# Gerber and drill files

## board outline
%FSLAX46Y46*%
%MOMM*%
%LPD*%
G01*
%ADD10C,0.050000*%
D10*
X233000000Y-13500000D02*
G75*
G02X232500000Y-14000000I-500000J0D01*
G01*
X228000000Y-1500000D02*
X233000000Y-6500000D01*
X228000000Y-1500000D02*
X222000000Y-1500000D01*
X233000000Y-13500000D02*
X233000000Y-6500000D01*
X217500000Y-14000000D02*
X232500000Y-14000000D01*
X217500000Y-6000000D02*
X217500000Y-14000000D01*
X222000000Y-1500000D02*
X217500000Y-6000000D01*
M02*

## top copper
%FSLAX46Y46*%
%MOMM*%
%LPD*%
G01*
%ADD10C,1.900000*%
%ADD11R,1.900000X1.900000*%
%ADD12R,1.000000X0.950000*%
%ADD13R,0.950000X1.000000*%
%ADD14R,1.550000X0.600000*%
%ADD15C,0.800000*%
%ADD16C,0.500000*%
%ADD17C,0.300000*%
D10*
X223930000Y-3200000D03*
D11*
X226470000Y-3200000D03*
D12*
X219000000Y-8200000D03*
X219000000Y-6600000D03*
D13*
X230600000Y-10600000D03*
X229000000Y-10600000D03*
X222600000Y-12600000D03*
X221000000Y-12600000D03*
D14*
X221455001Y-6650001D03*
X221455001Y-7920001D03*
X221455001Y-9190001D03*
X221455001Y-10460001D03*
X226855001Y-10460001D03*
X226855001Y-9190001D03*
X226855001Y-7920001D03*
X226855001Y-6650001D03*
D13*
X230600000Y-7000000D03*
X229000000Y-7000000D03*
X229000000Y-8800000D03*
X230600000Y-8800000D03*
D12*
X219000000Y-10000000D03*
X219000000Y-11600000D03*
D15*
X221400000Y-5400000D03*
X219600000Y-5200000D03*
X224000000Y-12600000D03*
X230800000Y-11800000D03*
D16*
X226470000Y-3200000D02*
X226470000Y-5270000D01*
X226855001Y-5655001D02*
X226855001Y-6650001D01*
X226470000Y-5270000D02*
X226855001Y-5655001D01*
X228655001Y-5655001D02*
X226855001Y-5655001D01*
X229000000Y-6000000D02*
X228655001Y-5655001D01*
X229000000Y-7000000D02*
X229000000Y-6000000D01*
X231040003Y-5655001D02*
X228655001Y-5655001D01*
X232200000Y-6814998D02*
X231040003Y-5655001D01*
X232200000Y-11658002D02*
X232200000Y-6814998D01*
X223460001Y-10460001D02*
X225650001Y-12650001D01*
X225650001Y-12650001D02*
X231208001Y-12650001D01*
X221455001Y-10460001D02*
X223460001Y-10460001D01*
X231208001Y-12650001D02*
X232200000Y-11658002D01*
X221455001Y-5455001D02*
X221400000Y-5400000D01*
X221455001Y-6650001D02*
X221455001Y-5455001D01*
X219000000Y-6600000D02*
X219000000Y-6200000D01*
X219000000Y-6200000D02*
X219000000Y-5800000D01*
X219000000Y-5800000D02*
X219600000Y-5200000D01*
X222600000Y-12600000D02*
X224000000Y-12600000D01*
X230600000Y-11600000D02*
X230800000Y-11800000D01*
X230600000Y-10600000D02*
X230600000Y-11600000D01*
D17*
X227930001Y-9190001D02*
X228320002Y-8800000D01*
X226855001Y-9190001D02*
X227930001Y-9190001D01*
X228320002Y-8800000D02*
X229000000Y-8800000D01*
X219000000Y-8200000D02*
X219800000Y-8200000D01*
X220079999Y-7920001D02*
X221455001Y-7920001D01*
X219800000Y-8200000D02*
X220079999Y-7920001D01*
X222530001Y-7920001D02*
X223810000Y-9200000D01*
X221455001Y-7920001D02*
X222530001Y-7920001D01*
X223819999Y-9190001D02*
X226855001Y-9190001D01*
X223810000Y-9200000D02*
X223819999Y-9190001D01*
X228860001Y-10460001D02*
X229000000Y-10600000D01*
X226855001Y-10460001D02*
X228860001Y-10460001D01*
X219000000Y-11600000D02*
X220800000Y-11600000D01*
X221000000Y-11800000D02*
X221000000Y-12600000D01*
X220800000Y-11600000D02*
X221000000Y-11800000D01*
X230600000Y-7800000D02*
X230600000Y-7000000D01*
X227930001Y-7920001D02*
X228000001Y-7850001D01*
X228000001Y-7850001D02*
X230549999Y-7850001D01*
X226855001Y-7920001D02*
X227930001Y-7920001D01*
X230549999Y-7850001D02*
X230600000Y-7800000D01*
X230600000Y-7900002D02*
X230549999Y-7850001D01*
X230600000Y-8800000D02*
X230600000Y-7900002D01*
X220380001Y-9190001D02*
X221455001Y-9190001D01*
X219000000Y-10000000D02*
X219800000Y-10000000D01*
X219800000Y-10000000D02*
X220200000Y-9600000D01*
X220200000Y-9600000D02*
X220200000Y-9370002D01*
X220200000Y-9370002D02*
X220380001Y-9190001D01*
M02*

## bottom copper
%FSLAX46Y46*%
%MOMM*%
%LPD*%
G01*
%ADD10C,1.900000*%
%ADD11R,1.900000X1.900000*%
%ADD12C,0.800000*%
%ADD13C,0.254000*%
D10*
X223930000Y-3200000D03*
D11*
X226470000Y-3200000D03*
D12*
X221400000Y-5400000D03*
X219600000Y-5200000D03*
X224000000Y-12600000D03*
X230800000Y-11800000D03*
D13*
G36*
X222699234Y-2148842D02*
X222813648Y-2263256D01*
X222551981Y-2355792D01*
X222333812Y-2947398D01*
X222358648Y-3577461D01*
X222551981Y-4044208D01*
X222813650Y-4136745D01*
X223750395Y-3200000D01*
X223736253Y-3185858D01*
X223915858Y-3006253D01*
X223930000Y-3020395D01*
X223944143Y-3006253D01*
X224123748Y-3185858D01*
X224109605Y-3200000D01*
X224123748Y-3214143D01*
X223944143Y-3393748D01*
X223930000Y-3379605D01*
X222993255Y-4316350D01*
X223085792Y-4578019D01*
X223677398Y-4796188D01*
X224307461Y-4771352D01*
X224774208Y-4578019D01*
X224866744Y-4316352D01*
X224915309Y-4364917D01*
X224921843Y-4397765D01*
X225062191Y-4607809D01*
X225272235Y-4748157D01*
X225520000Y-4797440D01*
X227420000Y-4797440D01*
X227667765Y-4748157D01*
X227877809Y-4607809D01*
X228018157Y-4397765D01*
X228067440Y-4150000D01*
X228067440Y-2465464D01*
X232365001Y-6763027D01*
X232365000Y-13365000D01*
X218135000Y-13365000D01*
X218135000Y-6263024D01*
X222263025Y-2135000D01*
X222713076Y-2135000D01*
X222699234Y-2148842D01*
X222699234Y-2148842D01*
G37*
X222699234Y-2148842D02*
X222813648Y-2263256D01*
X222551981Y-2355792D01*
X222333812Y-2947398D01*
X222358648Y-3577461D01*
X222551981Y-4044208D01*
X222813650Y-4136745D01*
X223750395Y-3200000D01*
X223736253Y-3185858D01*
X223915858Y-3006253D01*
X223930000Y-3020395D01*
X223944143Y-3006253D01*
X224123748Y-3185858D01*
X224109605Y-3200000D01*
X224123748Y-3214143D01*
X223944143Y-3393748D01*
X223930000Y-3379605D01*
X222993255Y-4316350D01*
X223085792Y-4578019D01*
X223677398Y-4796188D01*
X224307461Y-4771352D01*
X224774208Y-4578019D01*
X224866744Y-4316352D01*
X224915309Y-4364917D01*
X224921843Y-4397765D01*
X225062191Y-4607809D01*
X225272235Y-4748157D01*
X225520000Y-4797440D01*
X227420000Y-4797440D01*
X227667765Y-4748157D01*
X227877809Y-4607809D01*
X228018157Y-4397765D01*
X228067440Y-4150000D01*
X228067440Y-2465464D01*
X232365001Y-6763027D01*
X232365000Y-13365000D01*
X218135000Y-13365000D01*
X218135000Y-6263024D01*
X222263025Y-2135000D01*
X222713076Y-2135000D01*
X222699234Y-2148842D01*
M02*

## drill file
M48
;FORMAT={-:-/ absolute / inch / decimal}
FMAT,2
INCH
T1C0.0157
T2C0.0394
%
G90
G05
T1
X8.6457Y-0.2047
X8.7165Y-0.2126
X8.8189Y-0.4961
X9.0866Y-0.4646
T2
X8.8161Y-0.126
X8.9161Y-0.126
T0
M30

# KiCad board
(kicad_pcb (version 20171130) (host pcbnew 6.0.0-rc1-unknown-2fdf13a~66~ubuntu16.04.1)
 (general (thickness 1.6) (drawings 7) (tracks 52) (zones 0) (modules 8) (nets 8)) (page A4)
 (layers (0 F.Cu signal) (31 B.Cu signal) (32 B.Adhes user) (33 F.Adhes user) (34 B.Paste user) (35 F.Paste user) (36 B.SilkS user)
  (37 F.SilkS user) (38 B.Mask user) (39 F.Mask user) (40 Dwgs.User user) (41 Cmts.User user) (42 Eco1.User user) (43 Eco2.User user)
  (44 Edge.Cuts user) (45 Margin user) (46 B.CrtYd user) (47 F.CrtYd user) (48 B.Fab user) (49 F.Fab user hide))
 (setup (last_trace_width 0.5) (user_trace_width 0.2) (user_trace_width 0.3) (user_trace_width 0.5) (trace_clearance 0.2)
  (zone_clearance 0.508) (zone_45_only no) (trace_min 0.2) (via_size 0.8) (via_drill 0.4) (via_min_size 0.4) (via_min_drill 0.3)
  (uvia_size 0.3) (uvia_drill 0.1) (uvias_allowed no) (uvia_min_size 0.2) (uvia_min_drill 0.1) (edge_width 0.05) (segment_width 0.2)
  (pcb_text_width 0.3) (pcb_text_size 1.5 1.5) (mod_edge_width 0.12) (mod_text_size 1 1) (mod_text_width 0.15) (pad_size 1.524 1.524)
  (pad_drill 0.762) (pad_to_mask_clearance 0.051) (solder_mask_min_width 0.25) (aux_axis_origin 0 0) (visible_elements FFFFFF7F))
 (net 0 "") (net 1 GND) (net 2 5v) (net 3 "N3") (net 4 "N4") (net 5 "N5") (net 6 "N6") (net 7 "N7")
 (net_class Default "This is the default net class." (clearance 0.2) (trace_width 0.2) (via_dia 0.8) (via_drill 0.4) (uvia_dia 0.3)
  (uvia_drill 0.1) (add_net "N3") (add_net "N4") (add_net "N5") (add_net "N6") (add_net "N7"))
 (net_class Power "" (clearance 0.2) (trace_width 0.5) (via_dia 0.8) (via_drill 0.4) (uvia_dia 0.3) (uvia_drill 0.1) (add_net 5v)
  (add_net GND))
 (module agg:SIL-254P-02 (layer F.Cu) (at 225.2 3.2 180)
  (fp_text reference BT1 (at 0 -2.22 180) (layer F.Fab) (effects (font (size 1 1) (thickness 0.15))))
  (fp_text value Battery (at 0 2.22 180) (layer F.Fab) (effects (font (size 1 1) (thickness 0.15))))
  (pad 2 thru_hole circle (at 1.27 0 180) (size 1.9 1.9) (drill 1) (layers *.Cu *.Mask F.SilkS) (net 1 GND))
  (pad 1 thru_hole rect (at -1.27 0 180) (size 1.9 1.9) (drill 1) (layers *.Cu *.Mask F.SilkS) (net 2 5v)))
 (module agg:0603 (layer F.Cu) (at 219 7.4 270)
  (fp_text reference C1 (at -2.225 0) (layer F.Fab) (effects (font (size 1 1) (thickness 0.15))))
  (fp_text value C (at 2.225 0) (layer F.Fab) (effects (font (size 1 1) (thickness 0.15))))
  (pad 2 smd rect (at 0.8 0 270) (size 0.95 1) (layers F.Cu F.Paste F.Mask) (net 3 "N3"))
  (pad 1 smd rect (at -0.8 0 270) (size 0.95 1) (layers F.Cu F.Paste F.Mask) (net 1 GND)))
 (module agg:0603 (layer F.Cu) (at 229.8 10.6 180)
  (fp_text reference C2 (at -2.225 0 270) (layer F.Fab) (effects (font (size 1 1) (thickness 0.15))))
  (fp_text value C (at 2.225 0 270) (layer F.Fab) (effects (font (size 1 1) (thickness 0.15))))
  (pad 1 smd rect (at -0.8 0 180) (size 0.95 1) (layers F.Cu F.Paste F.Mask) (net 1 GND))
  (pad 2 smd rect (at 0.8 0 180) (size 0.95 1) (layers F.Cu F.Paste F.Mask) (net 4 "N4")))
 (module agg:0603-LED (layer F.Cu) (at 221.8 12.6 180)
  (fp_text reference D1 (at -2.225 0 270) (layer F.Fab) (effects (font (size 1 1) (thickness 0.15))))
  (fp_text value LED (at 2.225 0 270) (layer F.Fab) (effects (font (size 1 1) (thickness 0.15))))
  (pad 1 smd rect (at -0.8 0 180) (size 0.95 1) (layers F.Cu F.Paste F.Mask) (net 1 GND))
  (pad 2 smd rect (at 0.8 0 180) (size 0.95 1) (layers F.Cu F.Paste F.Mask) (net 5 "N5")))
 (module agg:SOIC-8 (layer F.Cu) (at 224.155001 8.555001)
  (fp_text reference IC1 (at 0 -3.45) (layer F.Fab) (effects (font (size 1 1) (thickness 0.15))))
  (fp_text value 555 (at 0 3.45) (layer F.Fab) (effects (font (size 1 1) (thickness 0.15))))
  (pad 1 smd rect (at -2.7 -1.905) (size 1.55 0.6) (layers F.Cu F.Paste F.Mask) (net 1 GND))
  (pad 2 smd rect (at -2.7 -0.635) (size 1.55 0.6) (layers F.Cu F.Paste F.Mask) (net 3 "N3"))
  (pad 3 smd rect (at -2.7 0.635) (size 1.55 0.6) (layers F.Cu F.Paste F.Mask) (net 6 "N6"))
  (pad 4 smd rect (at -2.7 1.905) (size 1.55 0.6) (layers F.Cu F.Paste F.Mask) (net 2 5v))
  (pad 5 smd rect (at 2.7 1.905) (size 1.55 0.6) (layers F.Cu F.Paste F.Mask) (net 4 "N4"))
  (pad 6 smd rect (at 2.7 0.635) (size 1.55 0.6) (layers F.Cu F.Paste F.Mask) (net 3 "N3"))
  (pad 7 smd rect (at 2.7 -0.635) (size 1.55 0.6) (layers F.Cu F.Paste F.Mask) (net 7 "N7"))
  (pad 8 smd rect (at 2.7 -1.905) (size 1.55 0.6) (layers F.Cu F.Paste F.Mask) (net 2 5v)))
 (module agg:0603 (layer F.Cu) (at 229.8 7)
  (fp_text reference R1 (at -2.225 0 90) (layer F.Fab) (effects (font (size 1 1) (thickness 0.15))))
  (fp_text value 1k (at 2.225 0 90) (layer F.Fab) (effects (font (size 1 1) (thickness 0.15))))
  (pad 2 smd rect (at 0.8 0) (size 0.95 1) (layers F.Cu F.Paste F.Mask) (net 7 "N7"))
  (pad 1 smd rect (at -0.8 0) (size 0.95 1) (layers F.Cu F.Paste F.Mask) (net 2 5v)))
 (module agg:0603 (layer F.Cu) (at 229.8 8.8)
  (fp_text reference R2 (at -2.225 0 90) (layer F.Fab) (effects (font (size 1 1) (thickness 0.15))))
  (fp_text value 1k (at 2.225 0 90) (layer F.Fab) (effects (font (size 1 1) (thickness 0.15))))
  (pad 1 smd rect (at -0.8 0) (size 0.95 1) (layers F.Cu F.Paste F.Mask) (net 3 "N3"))
  (pad 2 smd rect (at 0.8 0) (size 0.95 1) (layers F.Cu F.Paste F.Mask) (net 7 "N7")))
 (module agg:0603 (layer F.Cu) (at 219 10.8 270)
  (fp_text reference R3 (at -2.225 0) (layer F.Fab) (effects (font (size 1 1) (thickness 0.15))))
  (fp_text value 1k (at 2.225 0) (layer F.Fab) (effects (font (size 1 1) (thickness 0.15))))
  (pad 1 smd rect (at -0.8 0 270) (size 0.95 1) (layers F.Cu F.Paste F.Mask) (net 6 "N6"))
  (pad 2 smd rect (at 0.8 0 270) (size 0.95 1) (layers F.Cu F.Paste F.Mask) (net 5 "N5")))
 (gr_arc (start 232.5 13.5) (end 232.5 14) (angle -90) (layer Edge.Cuts) (width 0.05))
 (gr_line (start 228 1.5) (end 233 6.5) (layer Edge.Cuts) (width 0.05))
 (gr_line (start 228 1.5) (end 222 1.5) (layer Edge.Cuts) (width 0.05))
 (gr_line (start 233 13.5) (end 233 6.5) (layer Edge.Cuts) (width 0.05))
 (gr_line (start 217.5 14) (end 232.5 14) (layer Edge.Cuts) (width 0.05))
 (gr_line (start 217.5 6) (end 217.5 14) (layer Edge.Cuts) (width 0.05))
 (gr_line (start 222 1.5) (end 217.5 6) (layer Edge.Cuts) (width 0.05))
 (segment (start 226.47 3.2) (end 226.47 5.27) (width 0.5) (layer F.Cu) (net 2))
 (segment (start 226.855001 5.655001) (end 226.855001 6.650001) (width 0.5) (layer F.Cu) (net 2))
 (segment (start 226.47 5.27) (end 226.855001 5.655001) (width 0.5) (layer F.Cu) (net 2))
 (segment (start 228.655001 5.655001) (end 226.855001 5.655001) (width 0.5) (layer F.Cu) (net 2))
 (segment (start 229 6) (end 228.655001 5.655001) (width 0.5) (layer F.Cu) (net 2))
 (segment (start 229 7) (end 229 6) (width 0.5) (layer F.Cu) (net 2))
 (segment (start 231.040003 5.655001) (end 228.655001 5.655001) (width 0.5) (layer F.Cu) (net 2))
 (segment (start 232.2 6.814998) (end 231.040003 5.655001) (width 0.5) (layer F.Cu) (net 2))
 (segment (start 232.2 11.658002) (end 232.2 6.814998) (width 0.5) (layer F.Cu) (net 2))
 (segment (start 223.460001 10.460001) (end 225.650001 12.650001) (width 0.5) (layer F.Cu) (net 2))
 (segment (start 225.650001 12.650001) (end 231.208001 12.650001) (width 0.5) (layer F.Cu) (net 2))
 (segment (start 221.455001 10.460001) (end 223.460001 10.460001) (width 0.5) (layer F.Cu) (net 2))
 (segment (start 231.208001 12.650001) (end 232.2 11.658002) (width 0.5) (layer F.Cu) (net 2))
 (segment (start 221.455001 5.455001) (end 221.4 5.4) (width 0.5) (layer F.Cu) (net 1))
 (via (at 221.4 5.4) (size 0.8) (drill 0.4) (layers F.Cu B.Cu) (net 1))
 (segment (start 221.455001 6.650001) (end 221.455001 5.455001) (width 0.5) (layer F.Cu) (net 1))
 (segment (start 219 6.6) (end 219 6.2) (width 0.5) (layer F.Cu) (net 1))
 (segment (start 219 6.2) (end 219 5.8) (width 0.5) (layer F.Cu) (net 1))
 (segment (start 219 5.8) (end 219.6 5.2) (width 0.5) (layer F.Cu) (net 1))
 (via (at 219.6 5.2) (size 0.8) (drill 0.4) (layers F.Cu B.Cu) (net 1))
 (via (at 224 12.6) (size 0.8) (drill 0.4) (layers F.Cu B.Cu) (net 1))
 (segment (start 222.6 12.6) (end 224 12.6) (width 0.5) (layer F.Cu) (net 1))
 (via (at 230.8 11.8) (size 0.8) (drill 0.4) (layers F.Cu B.Cu) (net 1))
 (segment (start 230.6 11.6) (end 230.8 11.8) (width 0.5) (layer F.Cu) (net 1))
 (segment (start 230.6 10.6) (end 230.6 11.6) (width 0.5) (layer F.Cu) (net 1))
 (segment (start 227.930001 9.190001) (end 228.320002 8.8) (width 0.3) (layer F.Cu) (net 3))
 (segment (start 226.855001 9.190001) (end 227.930001 9.190001) (width 0.3) (layer F.Cu) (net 3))
 (segment (start 228.320002 8.8) (end 229 8.8) (width 0.3) (layer F.Cu) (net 3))
 (segment (start 219 8.2) (end 219.8 8.2) (width 0.3) (layer F.Cu) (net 3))
 (segment (start 220.079999 7.920001) (end 221.455001 7.920001) (width 0.3) (layer F.Cu) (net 3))
 (segment (start 219.8 8.2) (end 220.079999 7.920001) (width 0.3) (layer F.Cu) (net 3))
 (segment (start 222.530001 7.920001) (end 223.81 9.2) (width 0.3) (layer F.Cu) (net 3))
 (segment (start 221.455001 7.920001) (end 222.530001 7.920001) (width 0.3) (layer F.Cu) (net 3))
 (segment (start 223.819999 9.190001) (end 226.855001 9.190001) (width 0.3) (layer F.Cu) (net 3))
 (segment (start 223.81 9.2) (end 223.819999 9.190001) (width 0.3) (layer F.Cu) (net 3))
 (segment (start 228.860001 10.460001) (end 229 10.6) (width 0.3) (layer F.Cu) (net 4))
 (segment (start 226.855001 10.460001) (end 228.860001 10.460001) (width 0.3) (layer F.Cu) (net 4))
 (segment (start 219 11.6) (end 220.8 11.6) (width 0.3) (layer F.Cu) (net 5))
 (segment (start 221 11.8) (end 221 12.6) (width 0.3) (layer F.Cu) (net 5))
 (segment (start 220.8 11.6) (end 221 11.8) (width 0.3) (layer F.Cu) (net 5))
 (segment (start 230.6 7.8) (end 230.6 7) (width 0.3) (layer F.Cu) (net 7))
 (segment (start 227.930001 7.920001) (end 228.000001 7.850001) (width 0.3) (layer F.Cu) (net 7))
 (segment (start 228.000001 7.850001) (end 230.549999 7.850001) (width 0.3) (layer F.Cu) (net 7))
 (segment (start 226.855001 7.920001) (end 227.930001 7.920001) (width 0.3) (layer F.Cu) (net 7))
 (segment (start 230.549999 7.850001) (end 230.6 7.8) (width 0.3) (layer F.Cu) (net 7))
 (segment (start 230.6 7.900002) (end 230.549999 7.850001) (width 0.3) (layer F.Cu) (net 7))
 (segment (start 230.6 8.8) (end 230.6 7.900002) (width 0.3) (layer F.Cu) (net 7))
 (segment (start 220.380001 9.190001) (end 221.455001 9.190001) (width 0.3) (layer F.Cu) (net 6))
 (segment (start 219 10) (end 219.8 10) (width 0.3) (layer F.Cu) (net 6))
 (segment (start 219.8 10) (end 220.2 9.6) (width 0.3) (layer F.Cu) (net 6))
 (segment (start 220.2 9.6) (end 220.2 9.370002) (width 0.3) (layer F.Cu) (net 6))
 (segment (start 220.2 9.370002) (end 220.380001 9.190001) (width 0.3) (layer F.Cu) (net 6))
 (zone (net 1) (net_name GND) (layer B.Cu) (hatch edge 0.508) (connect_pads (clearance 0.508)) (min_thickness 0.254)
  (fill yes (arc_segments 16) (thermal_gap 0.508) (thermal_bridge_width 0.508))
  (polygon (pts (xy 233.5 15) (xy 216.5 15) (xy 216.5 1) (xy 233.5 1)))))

